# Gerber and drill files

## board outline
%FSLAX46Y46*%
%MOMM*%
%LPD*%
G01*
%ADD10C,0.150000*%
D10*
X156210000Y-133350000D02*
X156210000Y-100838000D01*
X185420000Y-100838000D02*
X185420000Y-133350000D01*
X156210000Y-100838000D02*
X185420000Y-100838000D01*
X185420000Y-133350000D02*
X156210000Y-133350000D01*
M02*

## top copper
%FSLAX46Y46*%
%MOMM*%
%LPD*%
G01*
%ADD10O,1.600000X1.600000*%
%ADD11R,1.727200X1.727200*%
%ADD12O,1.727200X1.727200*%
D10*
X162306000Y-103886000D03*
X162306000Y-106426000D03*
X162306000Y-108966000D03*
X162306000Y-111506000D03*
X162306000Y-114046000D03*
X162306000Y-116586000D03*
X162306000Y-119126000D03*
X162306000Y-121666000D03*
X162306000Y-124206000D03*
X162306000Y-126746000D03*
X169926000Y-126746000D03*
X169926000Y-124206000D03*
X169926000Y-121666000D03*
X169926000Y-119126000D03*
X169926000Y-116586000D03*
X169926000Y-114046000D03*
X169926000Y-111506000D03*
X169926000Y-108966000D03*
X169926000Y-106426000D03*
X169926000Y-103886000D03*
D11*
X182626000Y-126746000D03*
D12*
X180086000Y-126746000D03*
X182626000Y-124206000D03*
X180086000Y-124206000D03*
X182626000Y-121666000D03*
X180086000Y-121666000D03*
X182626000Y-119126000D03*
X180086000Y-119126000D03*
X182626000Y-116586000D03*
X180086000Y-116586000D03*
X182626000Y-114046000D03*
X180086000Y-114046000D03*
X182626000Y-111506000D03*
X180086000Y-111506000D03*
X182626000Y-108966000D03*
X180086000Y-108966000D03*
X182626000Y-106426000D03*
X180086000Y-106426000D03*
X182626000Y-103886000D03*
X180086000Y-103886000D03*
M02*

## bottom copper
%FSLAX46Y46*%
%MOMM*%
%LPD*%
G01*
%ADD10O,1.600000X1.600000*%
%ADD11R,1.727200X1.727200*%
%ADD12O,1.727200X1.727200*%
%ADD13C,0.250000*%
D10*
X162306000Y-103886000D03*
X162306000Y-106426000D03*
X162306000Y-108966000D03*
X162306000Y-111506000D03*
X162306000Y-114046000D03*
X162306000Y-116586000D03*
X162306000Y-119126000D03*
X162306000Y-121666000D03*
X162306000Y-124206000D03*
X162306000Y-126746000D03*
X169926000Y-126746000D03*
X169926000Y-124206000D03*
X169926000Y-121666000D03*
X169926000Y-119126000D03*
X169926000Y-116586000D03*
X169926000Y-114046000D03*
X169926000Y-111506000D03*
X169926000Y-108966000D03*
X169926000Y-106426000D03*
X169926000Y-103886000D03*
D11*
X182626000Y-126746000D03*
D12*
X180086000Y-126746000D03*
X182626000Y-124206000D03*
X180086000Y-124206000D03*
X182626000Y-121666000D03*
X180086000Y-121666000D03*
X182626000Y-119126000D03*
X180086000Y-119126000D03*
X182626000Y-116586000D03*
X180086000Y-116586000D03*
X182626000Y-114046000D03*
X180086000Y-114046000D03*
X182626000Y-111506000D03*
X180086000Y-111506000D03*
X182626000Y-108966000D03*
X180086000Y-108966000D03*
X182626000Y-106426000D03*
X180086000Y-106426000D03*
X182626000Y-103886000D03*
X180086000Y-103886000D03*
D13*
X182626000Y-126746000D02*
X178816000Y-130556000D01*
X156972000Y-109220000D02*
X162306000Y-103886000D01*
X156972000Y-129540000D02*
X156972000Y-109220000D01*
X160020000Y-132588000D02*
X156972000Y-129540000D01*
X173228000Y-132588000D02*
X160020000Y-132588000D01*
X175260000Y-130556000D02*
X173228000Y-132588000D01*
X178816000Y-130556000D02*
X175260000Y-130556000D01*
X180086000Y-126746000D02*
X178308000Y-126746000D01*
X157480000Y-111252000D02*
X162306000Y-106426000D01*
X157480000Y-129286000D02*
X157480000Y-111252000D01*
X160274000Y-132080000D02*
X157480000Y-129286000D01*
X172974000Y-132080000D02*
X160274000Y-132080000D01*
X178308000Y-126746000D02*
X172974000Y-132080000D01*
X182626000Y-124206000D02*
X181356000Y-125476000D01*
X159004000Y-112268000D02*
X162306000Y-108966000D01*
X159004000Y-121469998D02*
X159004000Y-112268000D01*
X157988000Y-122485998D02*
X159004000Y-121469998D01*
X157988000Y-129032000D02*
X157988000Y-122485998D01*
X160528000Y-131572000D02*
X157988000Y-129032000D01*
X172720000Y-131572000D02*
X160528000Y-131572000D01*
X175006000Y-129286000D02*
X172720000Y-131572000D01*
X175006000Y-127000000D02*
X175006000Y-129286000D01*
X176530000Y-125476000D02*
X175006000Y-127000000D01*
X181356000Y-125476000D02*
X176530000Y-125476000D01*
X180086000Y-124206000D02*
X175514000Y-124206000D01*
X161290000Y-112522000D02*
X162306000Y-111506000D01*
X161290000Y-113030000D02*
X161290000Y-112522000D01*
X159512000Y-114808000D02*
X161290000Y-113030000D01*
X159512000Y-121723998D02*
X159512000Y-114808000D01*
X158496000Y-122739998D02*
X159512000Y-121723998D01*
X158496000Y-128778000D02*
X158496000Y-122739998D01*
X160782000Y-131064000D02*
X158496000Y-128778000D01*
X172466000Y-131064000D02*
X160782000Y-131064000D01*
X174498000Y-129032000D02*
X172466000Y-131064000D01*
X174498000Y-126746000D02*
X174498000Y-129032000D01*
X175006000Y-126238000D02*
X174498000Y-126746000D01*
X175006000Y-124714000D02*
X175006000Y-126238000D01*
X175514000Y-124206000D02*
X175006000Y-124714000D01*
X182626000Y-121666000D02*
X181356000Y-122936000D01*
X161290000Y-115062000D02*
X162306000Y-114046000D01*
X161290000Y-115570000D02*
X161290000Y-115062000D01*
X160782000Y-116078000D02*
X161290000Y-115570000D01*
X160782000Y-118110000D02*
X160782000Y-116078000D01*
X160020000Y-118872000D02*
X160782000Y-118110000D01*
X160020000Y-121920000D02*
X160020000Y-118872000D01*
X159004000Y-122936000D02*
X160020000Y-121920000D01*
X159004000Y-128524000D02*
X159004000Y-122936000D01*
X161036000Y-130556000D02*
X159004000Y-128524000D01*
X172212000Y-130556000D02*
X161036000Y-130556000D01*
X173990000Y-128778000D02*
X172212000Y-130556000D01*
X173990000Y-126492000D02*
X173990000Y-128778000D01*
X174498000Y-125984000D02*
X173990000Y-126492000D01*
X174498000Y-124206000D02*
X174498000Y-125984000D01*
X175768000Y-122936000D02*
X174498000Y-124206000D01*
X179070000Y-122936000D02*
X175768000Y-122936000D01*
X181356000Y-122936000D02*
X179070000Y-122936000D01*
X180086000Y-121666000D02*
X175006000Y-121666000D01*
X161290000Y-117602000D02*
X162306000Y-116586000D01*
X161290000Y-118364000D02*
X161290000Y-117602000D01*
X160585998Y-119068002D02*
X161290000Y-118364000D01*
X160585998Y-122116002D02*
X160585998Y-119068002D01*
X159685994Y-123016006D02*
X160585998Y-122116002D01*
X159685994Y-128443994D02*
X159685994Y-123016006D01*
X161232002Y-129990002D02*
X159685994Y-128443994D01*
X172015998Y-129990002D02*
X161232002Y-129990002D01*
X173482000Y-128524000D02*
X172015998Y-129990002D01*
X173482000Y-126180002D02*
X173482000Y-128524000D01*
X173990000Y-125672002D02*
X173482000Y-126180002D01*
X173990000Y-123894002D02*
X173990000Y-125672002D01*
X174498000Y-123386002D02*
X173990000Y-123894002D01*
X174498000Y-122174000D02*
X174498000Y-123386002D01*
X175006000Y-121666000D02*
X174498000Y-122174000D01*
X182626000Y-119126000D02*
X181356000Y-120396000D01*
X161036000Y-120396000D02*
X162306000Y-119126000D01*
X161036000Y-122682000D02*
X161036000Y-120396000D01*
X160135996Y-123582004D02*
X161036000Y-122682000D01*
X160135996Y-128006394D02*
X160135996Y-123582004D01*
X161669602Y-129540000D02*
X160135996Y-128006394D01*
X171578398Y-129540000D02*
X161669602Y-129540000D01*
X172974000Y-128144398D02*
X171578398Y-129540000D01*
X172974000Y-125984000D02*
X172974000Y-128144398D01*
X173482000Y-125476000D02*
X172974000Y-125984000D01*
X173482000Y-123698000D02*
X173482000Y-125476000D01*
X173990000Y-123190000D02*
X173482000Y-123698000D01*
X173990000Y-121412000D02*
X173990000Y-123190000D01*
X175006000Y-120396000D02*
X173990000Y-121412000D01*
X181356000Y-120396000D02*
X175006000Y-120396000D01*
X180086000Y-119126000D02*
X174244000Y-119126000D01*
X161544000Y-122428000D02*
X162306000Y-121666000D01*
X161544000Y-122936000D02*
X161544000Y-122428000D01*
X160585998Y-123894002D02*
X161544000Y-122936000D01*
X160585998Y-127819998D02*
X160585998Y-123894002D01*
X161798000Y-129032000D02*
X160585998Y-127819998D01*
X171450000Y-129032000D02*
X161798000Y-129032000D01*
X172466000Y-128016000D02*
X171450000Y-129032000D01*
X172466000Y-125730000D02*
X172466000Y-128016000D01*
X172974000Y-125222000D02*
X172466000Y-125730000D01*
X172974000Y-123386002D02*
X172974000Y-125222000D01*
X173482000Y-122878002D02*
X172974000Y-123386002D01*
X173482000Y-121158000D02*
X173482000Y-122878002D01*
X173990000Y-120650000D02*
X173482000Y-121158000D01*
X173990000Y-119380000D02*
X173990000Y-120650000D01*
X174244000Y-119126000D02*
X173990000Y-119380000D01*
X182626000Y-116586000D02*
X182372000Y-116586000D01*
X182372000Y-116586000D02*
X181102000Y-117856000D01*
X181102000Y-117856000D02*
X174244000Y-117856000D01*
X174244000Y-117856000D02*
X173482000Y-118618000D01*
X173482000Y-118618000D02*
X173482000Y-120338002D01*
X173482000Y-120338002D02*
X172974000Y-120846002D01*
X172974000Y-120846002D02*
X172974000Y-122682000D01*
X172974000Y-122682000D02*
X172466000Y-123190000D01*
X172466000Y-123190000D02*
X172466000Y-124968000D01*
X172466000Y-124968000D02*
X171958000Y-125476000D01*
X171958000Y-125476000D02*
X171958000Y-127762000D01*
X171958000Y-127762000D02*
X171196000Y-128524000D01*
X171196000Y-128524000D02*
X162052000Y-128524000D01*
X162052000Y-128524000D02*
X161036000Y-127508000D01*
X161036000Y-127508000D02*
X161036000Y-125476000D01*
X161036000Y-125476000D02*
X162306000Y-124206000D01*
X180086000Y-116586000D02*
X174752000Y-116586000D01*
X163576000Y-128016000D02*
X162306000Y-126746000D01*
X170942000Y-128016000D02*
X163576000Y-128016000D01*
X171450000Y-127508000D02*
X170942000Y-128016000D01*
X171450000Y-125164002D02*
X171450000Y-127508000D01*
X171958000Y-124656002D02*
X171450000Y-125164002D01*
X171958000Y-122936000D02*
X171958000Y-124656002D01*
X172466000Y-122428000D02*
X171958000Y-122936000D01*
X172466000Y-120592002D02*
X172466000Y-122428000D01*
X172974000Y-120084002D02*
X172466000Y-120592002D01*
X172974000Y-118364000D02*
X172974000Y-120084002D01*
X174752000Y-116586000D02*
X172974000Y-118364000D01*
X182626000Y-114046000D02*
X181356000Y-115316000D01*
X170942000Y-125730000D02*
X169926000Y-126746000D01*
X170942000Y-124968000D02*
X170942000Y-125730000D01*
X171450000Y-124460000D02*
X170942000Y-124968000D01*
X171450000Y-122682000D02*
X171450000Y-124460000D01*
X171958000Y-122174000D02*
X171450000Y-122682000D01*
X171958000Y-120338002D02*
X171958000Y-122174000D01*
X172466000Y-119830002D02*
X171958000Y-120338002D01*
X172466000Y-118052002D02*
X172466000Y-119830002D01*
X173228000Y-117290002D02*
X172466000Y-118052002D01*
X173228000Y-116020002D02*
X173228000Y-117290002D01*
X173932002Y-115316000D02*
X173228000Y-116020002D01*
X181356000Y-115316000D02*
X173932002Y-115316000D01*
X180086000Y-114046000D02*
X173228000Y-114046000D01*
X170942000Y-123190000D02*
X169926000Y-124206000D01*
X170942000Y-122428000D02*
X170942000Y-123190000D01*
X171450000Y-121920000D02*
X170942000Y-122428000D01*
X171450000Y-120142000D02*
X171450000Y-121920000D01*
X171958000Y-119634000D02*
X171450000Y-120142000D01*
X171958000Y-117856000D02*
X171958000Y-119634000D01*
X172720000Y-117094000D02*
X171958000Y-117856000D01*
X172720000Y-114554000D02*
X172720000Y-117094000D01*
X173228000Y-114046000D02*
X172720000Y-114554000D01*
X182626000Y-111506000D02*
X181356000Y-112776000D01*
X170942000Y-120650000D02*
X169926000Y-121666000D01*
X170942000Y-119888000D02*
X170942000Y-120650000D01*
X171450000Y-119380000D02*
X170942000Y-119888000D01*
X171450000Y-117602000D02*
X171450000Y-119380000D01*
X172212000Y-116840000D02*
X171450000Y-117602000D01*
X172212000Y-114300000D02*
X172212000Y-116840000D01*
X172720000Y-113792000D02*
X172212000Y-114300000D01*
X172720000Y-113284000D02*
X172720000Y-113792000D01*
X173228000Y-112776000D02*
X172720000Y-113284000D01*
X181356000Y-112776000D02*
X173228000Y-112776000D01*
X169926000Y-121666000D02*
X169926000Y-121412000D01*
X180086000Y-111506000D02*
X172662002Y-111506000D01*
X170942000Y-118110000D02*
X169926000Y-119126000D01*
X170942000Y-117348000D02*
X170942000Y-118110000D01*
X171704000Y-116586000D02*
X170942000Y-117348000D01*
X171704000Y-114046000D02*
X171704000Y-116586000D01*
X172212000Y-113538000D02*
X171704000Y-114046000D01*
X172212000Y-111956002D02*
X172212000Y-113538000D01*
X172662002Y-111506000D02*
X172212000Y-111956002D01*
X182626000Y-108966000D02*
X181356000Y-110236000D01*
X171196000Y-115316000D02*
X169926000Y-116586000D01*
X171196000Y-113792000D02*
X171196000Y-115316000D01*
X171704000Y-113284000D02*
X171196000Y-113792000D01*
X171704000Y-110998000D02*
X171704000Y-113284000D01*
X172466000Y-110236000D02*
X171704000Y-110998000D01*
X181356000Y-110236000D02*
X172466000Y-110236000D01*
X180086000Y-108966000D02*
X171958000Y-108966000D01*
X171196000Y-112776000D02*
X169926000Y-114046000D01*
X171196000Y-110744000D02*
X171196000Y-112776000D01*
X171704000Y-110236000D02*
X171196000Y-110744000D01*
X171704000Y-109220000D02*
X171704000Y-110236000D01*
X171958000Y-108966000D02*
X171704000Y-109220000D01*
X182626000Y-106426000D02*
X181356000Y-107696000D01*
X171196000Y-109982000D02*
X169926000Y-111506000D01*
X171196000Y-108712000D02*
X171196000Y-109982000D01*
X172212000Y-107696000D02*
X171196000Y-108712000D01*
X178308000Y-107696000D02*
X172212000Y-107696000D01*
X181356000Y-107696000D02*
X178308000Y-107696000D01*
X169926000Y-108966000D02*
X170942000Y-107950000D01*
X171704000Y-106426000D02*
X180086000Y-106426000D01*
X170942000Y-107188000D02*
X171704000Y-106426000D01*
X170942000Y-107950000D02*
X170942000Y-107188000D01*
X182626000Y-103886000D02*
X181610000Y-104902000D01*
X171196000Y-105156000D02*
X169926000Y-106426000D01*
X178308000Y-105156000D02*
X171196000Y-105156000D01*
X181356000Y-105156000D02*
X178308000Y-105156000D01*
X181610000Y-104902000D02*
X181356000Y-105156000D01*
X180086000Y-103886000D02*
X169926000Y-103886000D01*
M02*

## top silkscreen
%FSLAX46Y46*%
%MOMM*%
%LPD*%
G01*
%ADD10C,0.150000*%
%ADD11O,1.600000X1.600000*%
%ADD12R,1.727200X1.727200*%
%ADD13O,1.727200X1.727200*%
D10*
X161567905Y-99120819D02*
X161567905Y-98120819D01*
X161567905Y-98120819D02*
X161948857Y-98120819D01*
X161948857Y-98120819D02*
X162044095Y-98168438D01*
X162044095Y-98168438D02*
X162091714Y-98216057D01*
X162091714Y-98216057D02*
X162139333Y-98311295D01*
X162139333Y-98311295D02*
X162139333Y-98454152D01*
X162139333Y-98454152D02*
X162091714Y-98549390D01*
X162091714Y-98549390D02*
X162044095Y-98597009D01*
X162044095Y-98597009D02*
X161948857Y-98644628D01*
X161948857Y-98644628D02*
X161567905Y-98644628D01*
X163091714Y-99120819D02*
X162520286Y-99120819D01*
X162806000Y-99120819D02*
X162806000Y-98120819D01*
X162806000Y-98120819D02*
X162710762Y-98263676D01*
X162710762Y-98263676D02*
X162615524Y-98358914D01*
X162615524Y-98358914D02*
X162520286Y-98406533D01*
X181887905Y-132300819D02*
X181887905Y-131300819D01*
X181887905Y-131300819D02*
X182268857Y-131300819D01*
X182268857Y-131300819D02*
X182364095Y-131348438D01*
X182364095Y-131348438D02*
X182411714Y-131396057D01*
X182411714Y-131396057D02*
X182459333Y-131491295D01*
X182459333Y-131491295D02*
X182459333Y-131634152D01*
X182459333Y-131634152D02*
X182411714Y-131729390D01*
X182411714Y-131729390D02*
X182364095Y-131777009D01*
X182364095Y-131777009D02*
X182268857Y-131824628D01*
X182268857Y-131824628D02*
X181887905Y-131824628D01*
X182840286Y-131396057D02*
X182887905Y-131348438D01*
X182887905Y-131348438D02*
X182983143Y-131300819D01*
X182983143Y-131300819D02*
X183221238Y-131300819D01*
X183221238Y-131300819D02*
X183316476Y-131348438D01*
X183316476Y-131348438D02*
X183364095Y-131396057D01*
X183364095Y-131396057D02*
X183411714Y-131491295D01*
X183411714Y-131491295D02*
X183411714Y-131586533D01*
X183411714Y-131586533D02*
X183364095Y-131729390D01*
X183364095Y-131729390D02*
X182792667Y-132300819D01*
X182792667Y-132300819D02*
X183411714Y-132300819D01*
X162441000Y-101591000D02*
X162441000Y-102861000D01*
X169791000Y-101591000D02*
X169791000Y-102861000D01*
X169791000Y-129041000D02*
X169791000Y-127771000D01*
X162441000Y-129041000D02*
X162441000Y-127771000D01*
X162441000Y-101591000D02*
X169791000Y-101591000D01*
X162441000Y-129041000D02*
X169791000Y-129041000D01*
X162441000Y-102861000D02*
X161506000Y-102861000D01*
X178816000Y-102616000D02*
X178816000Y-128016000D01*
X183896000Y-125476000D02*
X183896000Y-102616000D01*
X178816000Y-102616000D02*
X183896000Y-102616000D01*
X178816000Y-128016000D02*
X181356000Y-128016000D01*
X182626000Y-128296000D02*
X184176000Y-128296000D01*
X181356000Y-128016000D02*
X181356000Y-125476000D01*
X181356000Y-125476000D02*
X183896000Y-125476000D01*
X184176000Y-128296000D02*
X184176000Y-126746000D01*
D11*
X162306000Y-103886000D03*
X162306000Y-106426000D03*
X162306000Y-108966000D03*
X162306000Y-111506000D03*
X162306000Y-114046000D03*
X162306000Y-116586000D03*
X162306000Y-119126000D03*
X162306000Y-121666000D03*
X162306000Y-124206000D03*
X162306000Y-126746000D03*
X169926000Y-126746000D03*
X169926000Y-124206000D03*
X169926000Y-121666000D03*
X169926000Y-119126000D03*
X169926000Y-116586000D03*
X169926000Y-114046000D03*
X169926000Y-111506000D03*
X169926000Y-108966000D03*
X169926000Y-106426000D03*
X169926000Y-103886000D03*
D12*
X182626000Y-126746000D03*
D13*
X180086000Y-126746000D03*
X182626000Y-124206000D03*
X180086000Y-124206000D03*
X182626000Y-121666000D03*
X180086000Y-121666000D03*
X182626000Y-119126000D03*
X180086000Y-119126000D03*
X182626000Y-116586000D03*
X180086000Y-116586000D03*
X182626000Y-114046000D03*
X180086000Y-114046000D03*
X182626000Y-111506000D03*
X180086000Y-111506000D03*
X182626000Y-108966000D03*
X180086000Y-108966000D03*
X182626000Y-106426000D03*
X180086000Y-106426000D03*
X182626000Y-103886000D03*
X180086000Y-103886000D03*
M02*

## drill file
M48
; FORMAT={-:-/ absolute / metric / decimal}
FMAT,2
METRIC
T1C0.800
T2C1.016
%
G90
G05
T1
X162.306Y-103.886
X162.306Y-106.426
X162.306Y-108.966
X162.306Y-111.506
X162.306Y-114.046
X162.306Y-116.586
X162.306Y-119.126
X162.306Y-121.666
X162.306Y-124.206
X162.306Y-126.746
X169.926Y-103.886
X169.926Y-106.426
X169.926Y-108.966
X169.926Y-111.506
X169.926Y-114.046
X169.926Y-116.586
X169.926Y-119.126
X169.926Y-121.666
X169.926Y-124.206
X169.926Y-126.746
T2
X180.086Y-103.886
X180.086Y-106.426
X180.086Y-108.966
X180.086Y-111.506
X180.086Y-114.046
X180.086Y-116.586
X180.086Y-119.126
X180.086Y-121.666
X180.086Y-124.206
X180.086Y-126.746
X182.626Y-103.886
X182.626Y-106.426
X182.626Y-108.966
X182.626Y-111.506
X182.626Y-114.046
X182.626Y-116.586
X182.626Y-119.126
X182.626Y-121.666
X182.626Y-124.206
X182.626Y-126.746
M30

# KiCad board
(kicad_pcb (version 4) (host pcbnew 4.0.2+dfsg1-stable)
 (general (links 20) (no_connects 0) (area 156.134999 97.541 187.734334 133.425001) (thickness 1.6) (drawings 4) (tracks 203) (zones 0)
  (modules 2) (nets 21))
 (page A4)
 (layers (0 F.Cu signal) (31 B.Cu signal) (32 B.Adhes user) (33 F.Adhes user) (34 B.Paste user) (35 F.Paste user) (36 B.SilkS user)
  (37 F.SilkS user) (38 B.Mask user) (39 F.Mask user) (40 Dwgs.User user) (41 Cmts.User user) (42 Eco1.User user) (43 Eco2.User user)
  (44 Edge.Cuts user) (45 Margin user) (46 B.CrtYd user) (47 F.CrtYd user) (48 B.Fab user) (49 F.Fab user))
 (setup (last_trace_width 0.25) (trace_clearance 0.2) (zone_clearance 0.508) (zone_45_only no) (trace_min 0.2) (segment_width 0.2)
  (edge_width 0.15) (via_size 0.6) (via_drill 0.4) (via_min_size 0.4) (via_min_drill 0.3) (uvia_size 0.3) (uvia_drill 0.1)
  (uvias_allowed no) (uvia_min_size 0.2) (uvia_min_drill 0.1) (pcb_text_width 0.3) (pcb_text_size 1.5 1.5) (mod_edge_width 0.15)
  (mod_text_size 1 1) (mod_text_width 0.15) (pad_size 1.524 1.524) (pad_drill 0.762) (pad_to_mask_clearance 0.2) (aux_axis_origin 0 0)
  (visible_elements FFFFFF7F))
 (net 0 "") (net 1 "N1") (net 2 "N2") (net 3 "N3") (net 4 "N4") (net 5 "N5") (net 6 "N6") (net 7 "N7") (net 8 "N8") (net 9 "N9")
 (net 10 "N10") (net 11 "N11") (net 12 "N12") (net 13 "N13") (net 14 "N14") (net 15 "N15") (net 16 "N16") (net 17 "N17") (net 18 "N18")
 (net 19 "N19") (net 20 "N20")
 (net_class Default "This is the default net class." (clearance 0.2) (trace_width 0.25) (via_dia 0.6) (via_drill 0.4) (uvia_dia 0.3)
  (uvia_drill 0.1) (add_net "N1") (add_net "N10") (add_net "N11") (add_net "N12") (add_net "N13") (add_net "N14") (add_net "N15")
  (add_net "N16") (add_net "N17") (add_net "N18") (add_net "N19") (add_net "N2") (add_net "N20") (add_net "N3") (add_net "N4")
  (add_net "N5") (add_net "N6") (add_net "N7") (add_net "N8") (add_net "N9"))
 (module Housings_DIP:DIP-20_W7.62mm (layer F.Cu) (at 162.306 103.886)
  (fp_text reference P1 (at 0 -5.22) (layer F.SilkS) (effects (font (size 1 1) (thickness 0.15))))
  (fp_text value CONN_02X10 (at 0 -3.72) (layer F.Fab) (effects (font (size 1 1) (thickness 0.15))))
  (fp_line (start 0.135 -2.295) (end 0.135 -1.025) (layer F.SilkS) (width 0.15))
  (fp_line (start 7.485 -2.295) (end 7.485 -1.025) (layer F.SilkS) (width 0.15))
  (fp_line (start 7.485 25.155) (end 7.485 23.885) (layer F.SilkS) (width 0.15))
  (fp_line (start 0.135 25.155) (end 0.135 23.885) (layer F.SilkS) (width 0.15))
  (fp_line (start 0.135 -2.295) (end 7.485 -2.295) (layer F.SilkS) (width 0.15))
  (fp_line (start 0.135 25.155) (end 7.485 25.155) (layer F.SilkS) (width 0.15))
  (fp_line (start 0.135 -1.025) (end -0.8 -1.025) (layer F.SilkS) (width 0.15))
  (pad 1 thru_hole oval (at 0 0) (size 1.6 1.6) (drill 0.8) (layers *.Cu *.Mask F.SilkS) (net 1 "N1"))
  (pad 2 thru_hole oval (at 0 2.54) (size 1.6 1.6) (drill 0.8) (layers *.Cu *.Mask F.SilkS) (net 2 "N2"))
  (pad 3 thru_hole oval (at 0 5.08) (size 1.6 1.6) (drill 0.8) (layers *.Cu *.Mask F.SilkS) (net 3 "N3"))
  (pad 4 thru_hole oval (at 0 7.62) (size 1.6 1.6) (drill 0.8) (layers *.Cu *.Mask F.SilkS) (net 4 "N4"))
  (pad 5 thru_hole oval (at 0 10.16) (size 1.6 1.6) (drill 0.8) (layers *.Cu *.Mask F.SilkS) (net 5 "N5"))
  (pad 6 thru_hole oval (at 0 12.7) (size 1.6 1.6) (drill 0.8) (layers *.Cu *.Mask F.SilkS) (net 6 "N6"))
  (pad 7 thru_hole oval (at 0 15.24) (size 1.6 1.6) (drill 0.8) (layers *.Cu *.Mask F.SilkS) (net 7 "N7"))
  (pad 8 thru_hole oval (at 0 17.78) (size 1.6 1.6) (drill 0.8) (layers *.Cu *.Mask F.SilkS) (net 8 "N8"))
  (pad 9 thru_hole oval (at 0 20.32) (size 1.6 1.6) (drill 0.8) (layers *.Cu *.Mask F.SilkS) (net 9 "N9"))
  (pad 10 thru_hole oval (at 0 22.86) (size 1.6 1.6) (drill 0.8) (layers *.Cu *.Mask F.SilkS) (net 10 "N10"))
  (pad 11 thru_hole oval (at 7.62 22.86) (size 1.6 1.6) (drill 0.8) (layers *.Cu *.Mask F.SilkS) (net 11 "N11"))
  (pad 12 thru_hole oval (at 7.62 20.32) (size 1.6 1.6) (drill 0.8) (layers *.Cu *.Mask F.SilkS) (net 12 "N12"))
  (pad 13 thru_hole oval (at 7.62 17.78) (size 1.6 1.6) (drill 0.8) (layers *.Cu *.Mask F.SilkS) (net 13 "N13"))
  (pad 14 thru_hole oval (at 7.62 15.24) (size 1.6 1.6) (drill 0.8) (layers *.Cu *.Mask F.SilkS) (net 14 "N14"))
  (pad 15 thru_hole oval (at 7.62 12.7) (size 1.6 1.6) (drill 0.8) (layers *.Cu *.Mask F.SilkS) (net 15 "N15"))
  (pad 16 thru_hole oval (at 7.62 10.16) (size 1.6 1.6) (drill 0.8) (layers *.Cu *.Mask F.SilkS) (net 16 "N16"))
  (pad 17 thru_hole oval (at 7.62 7.62) (size 1.6 1.6) (drill 0.8) (layers *.Cu *.Mask F.SilkS) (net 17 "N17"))
  (pad 18 thru_hole oval (at 7.62 5.08) (size 1.6 1.6) (drill 0.8) (layers *.Cu *.Mask F.SilkS) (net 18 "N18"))
  (pad 19 thru_hole oval (at 7.62 2.54) (size 1.6 1.6) (drill 0.8) (layers *.Cu *.Mask F.SilkS) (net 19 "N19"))
  (pad 20 thru_hole oval (at 7.62 0) (size 1.6 1.6) (drill 0.8) (layers *.Cu *.Mask F.SilkS) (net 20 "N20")))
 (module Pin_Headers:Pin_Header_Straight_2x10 (layer F.Cu) (at 182.626 126.746 180)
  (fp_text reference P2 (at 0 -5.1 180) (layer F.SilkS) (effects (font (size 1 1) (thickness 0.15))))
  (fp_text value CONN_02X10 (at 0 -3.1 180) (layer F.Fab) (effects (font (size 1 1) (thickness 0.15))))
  (fp_line (start 3.81 24.13) (end 3.81 -1.27) (layer F.SilkS) (width 0.15))
  (fp_line (start -1.27 1.27) (end -1.27 24.13) (layer F.SilkS) (width 0.15))
  (fp_line (start 3.81 24.13) (end -1.27 24.13) (layer F.SilkS) (width 0.15))
  (fp_line (start 3.81 -1.27) (end 1.27 -1.27) (layer F.SilkS) (width 0.15))
  (fp_line (start 0 -1.55) (end -1.55 -1.55) (layer F.SilkS) (width 0.15))
  (fp_line (start 1.27 -1.27) (end 1.27 1.27) (layer F.SilkS) (width 0.15))
  (fp_line (start 1.27 1.27) (end -1.27 1.27) (layer F.SilkS) (width 0.15))
  (fp_line (start -1.55 -1.55) (end -1.55 0) (layer F.SilkS) (width 0.15))
  (pad 1 thru_hole rect (at 0 0 180) (size 1.7272 1.7272) (drill 1.016) (layers *.Cu *.Mask F.SilkS) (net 1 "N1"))
  (pad 2 thru_hole oval (at 2.54 0 180) (size 1.7272 1.7272) (drill 1.016) (layers *.Cu *.Mask F.SilkS) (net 2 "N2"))
  (pad 3 thru_hole oval (at 0 2.54 180) (size 1.7272 1.7272) (drill 1.016) (layers *.Cu *.Mask F.SilkS) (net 3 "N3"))
  (pad 4 thru_hole oval (at 2.54 2.54 180) (size 1.7272 1.7272) (drill 1.016) (layers *.Cu *.Mask F.SilkS) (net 4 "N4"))
  (pad 5 thru_hole oval (at 0 5.08 180) (size 1.7272 1.7272) (drill 1.016) (layers *.Cu *.Mask F.SilkS) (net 5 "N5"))
  (pad 6 thru_hole oval (at 2.54 5.08 180) (size 1.7272 1.7272) (drill 1.016) (layers *.Cu *.Mask F.SilkS) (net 6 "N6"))
  (pad 7 thru_hole oval (at 0 7.62 180) (size 1.7272 1.7272) (drill 1.016) (layers *.Cu *.Mask F.SilkS) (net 7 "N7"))
  (pad 8 thru_hole oval (at 2.54 7.62 180) (size 1.7272 1.7272) (drill 1.016) (layers *.Cu *.Mask F.SilkS) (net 8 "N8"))
  (pad 9 thru_hole oval (at 0 10.16 180) (size 1.7272 1.7272) (drill 1.016) (layers *.Cu *.Mask F.SilkS) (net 9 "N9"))
  (pad 10 thru_hole oval (at 2.54 10.16 180) (size 1.7272 1.7272) (drill 1.016) (layers *.Cu *.Mask F.SilkS) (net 10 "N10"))
  (pad 11 thru_hole oval (at 0 12.7 180) (size 1.7272 1.7272) (drill 1.016) (layers *.Cu *.Mask F.SilkS) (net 11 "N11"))
  (pad 12 thru_hole oval (at 2.54 12.7 180) (size 1.7272 1.7272) (drill 1.016) (layers *.Cu *.Mask F.SilkS) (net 12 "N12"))
  (pad 13 thru_hole oval (at 0 15.24 180) (size 1.7272 1.7272) (drill 1.016) (layers *.Cu *.Mask F.SilkS) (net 13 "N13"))
  (pad 14 thru_hole oval (at 2.54 15.24 180) (size 1.7272 1.7272) (drill 1.016) (layers *.Cu *.Mask F.SilkS) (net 14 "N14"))
  (pad 15 thru_hole oval (at 0 17.78 180) (size 1.7272 1.7272) (drill 1.016) (layers *.Cu *.Mask F.SilkS) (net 15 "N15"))
  (pad 16 thru_hole oval (at 2.54 17.78 180) (size 1.7272 1.7272) (drill 1.016) (layers *.Cu *.Mask F.SilkS) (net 16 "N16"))
  (pad 17 thru_hole oval (at 0 20.32 180) (size 1.7272 1.7272) (drill 1.016) (layers *.Cu *.Mask F.SilkS) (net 17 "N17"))
  (pad 18 thru_hole oval (at 2.54 20.32 180) (size 1.7272 1.7272) (drill 1.016) (layers *.Cu *.Mask F.SilkS) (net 18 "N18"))
  (pad 19 thru_hole oval (at 0 22.86 180) (size 1.7272 1.7272) (drill 1.016) (layers *.Cu *.Mask F.SilkS) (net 19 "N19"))
  (pad 20 thru_hole oval (at 2.54 22.86 180) (size 1.7272 1.7272) (drill 1.016) (layers *.Cu *.Mask F.SilkS) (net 20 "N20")))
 (gr_line (start 156.21 133.35) (end 156.21 100.838) (angle 90) (layer Edge.Cuts) (width 0.15))
 (gr_line (start 185.42 100.838) (end 185.42 133.35) (angle 90) (layer Edge.Cuts) (width 0.15))
 (gr_line (start 156.21 100.838) (end 185.42 100.838) (angle 90) (layer Edge.Cuts) (width 0.15))
 (gr_line (start 185.42 133.35) (end 156.21 133.35) (angle 90) (layer Edge.Cuts) (width 0.15))
 (segment (start 182.626 126.746) (end 178.816 130.556) (width 0.25) (layer B.Cu) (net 1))
 (segment (start 156.972 109.22) (end 162.306 103.886) (width 0.25) (layer B.Cu) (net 1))
 (segment (start 156.972 129.54) (end 156.972 109.22) (width 0.25) (layer B.Cu) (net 1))
 (segment (start 160.02 132.588) (end 156.972 129.54) (width 0.25) (layer B.Cu) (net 1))
 (segment (start 173.228 132.588) (end 160.02 132.588) (width 0.25) (layer B.Cu) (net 1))
 (segment (start 175.26 130.556) (end 173.228 132.588) (width 0.25) (layer B.Cu) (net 1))
 (segment (start 178.816 130.556) (end 175.26 130.556) (width 0.25) (layer B.Cu) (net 1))
 (segment (start 180.086 126.746) (end 178.308 126.746) (width 0.25) (layer B.Cu) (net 2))
 (segment (start 157.48 111.252) (end 162.306 106.426) (width 0.25) (layer B.Cu) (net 2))
 (segment (start 157.48 129.286) (end 157.48 111.252) (width 0.25) (layer B.Cu) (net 2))
 (segment (start 160.274 132.08) (end 157.48 129.286) (width 0.25) (layer B.Cu) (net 2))
 (segment (start 172.974 132.08) (end 160.274 132.08) (width 0.25) (layer B.Cu) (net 2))
 (segment (start 178.308 126.746) (end 172.974 132.08) (width 0.25) (layer B.Cu) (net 2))
 (segment (start 182.626 124.206) (end 181.356 125.476) (width 0.25) (layer B.Cu) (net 3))
 (segment (start 159.004 112.268) (end 162.306 108.966) (width 0.25) (layer B.Cu) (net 3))
 (segment (start 159.004 121.469998) (end 159.004 112.268) (width 0.25) (layer B.Cu) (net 3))
 (segment (start 157.988 122.485998) (end 159.004 121.469998) (width 0.25) (layer B.Cu) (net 3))
 (segment (start 157.988 129.032) (end 157.988 122.485998) (width 0.25) (layer B.Cu) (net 3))
 (segment (start 160.528 131.572) (end 157.988 129.032) (width 0.25) (layer B.Cu) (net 3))
 (segment (start 172.72 131.572) (end 160.528 131.572) (width 0.25) (layer B.Cu) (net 3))
 (segment (start 175.006 129.286) (end 172.72 131.572) (width 0.25) (layer B.Cu) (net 3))
 (segment (start 175.006 127) (end 175.006 129.286) (width 0.25) (layer B.Cu) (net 3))
 (segment (start 176.53 125.476) (end 175.006 127) (width 0.25) (layer B.Cu) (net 3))
 (segment (start 181.356 125.476) (end 176.53 125.476) (width 0.25) (layer B.Cu) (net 3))
 (segment (start 180.086 124.206) (end 175.514 124.206) (width 0.25) (layer B.Cu) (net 4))
 (segment (start 161.29 112.522) (end 162.306 111.506) (width 0.25) (layer B.Cu) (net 4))
 (segment (start 161.29 113.03) (end 161.29 112.522) (width 0.25) (layer B.Cu) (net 4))
 (segment (start 159.512 114.808) (end 161.29 113.03) (width 0.25) (layer B.Cu) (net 4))
 (segment (start 159.512 121.723998) (end 159.512 114.808) (width 0.25) (layer B.Cu) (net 4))
 (segment (start 158.496 122.739998) (end 159.512 121.723998) (width 0.25) (layer B.Cu) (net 4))
 (segment (start 158.496 128.778) (end 158.496 122.739998) (width 0.25) (layer B.Cu) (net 4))
 (segment (start 160.782 131.064) (end 158.496 128.778) (width 0.25) (layer B.Cu) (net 4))
 (segment (start 172.466 131.064) (end 160.782 131.064) (width 0.25) (layer B.Cu) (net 4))
 (segment (start 174.498 129.032) (end 172.466 131.064) (width 0.25) (layer B.Cu) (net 4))
 (segment (start 174.498 126.746) (end 174.498 129.032) (width 0.25) (layer B.Cu) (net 4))
 (segment (start 175.006 126.238) (end 174.498 126.746) (width 0.25) (layer B.Cu) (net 4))
 (segment (start 175.006 124.714) (end 175.006 126.238) (width 0.25) (layer B.Cu) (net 4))
 (segment (start 175.514 124.206) (end 175.006 124.714) (width 0.25) (layer B.Cu) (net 4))
 (segment (start 182.626 121.666) (end 181.356 122.936) (width 0.25) (layer B.Cu) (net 5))
 (segment (start 161.29 115.062) (end 162.306 114.046) (width 0.25) (layer B.Cu) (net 5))
 (segment (start 161.29 115.57) (end 161.29 115.062) (width 0.25) (layer B.Cu) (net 5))
 (segment (start 160.782 116.078) (end 161.29 115.57) (width 0.25) (layer B.Cu) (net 5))
 (segment (start 160.782 118.11) (end 160.782 116.078) (width 0.25) (layer B.Cu) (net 5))
 (segment (start 160.02 118.872) (end 160.782 118.11) (width 0.25) (layer B.Cu) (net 5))
 (segment (start 160.02 121.92) (end 160.02 118.872) (width 0.25) (layer B.Cu) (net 5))
 (segment (start 159.004 122.936) (end 160.02 121.92) (width 0.25) (layer B.Cu) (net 5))
 (segment (start 159.004 128.524) (end 159.004 122.936) (width 0.25) (layer B.Cu) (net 5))
 (segment (start 161.036 130.556) (end 159.004 128.524) (width 0.25) (layer B.Cu) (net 5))
 (segment (start 172.212 130.556) (end 161.036 130.556) (width 0.25) (layer B.Cu) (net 5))
 (segment (start 173.99 128.778) (end 172.212 130.556) (width 0.25) (layer B.Cu) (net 5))
 (segment (start 173.99 126.492) (end 173.99 128.778) (width 0.25) (layer B.Cu) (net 5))
 (segment (start 174.498 125.984) (end 173.99 126.492) (width 0.25) (layer B.Cu) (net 5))
 (segment (start 174.498 124.206) (end 174.498 125.984) (width 0.25) (layer B.Cu) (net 5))
 (segment (start 175.768 122.936) (end 174.498 124.206) (width 0.25) (layer B.Cu) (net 5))
 (segment (start 179.07 122.936) (end 175.768 122.936) (width 0.25) (layer B.Cu) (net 5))
 (segment (start 181.356 122.936) (end 179.07 122.936) (width 0.25) (layer B.Cu) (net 5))
 (segment (start 180.086 121.666) (end 175.006 121.666) (width 0.25) (layer B.Cu) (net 6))
 (segment (start 161.29 117.602) (end 162.306 116.586) (width 0.25) (layer B.Cu) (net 6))
 (segment (start 161.29 118.364) (end 161.29 117.602) (width 0.25) (layer B.Cu) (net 6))
 (segment (start 160.585998 119.068002) (end 161.29 118.364) (width 0.25) (layer B.Cu) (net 6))
 (segment (start 160.585998 122.116002) (end 160.585998 119.068002) (width 0.25) (layer B.Cu) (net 6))
 (segment (start 159.685994 123.016006) (end 160.585998 122.116002) (width 0.25) (layer B.Cu) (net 6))
 (segment (start 159.685994 128.443994) (end 159.685994 123.016006) (width 0.25) (layer B.Cu) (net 6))
 (segment (start 161.232002 129.990002) (end 159.685994 128.443994) (width 0.25) (layer B.Cu) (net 6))
 (segment (start 172.015998 129.990002) (end 161.232002 129.990002) (width 0.25) (layer B.Cu) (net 6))
 (segment (start 173.482 128.524) (end 172.015998 129.990002) (width 0.25) (layer B.Cu) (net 6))
 (segment (start 173.482 126.180002) (end 173.482 128.524) (width 0.25) (layer B.Cu) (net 6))
 (segment (start 173.99 125.672002) (end 173.482 126.180002) (width 0.25) (layer B.Cu) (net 6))
 (segment (start 173.99 123.894002) (end 173.99 125.672002) (width 0.25) (layer B.Cu) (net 6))
 (segment (start 174.498 123.386002) (end 173.99 123.894002) (width 0.25) (layer B.Cu) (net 6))
 (segment (start 174.498 122.174) (end 174.498 123.386002) (width 0.25) (layer B.Cu) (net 6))
 (segment (start 175.006 121.666) (end 174.498 122.174) (width 0.25) (layer B.Cu) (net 6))
 (segment (start 182.626 119.126) (end 181.356 120.396) (width 0.25) (layer B.Cu) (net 7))
 (segment (start 161.036 120.396) (end 162.306 119.126) (width 0.25) (layer B.Cu) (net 7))
 (segment (start 161.036 122.682) (end 161.036 120.396) (width 0.25) (layer B.Cu) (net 7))
 (segment (start 160.135996 123.582004) (end 161.036 122.682) (width 0.25) (layer B.Cu) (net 7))
 (segment (start 160.135996 128.006394) (end 160.135996 123.582004) (width 0.25) (layer B.Cu) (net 7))
 (segment (start 161.669602 129.54) (end 160.135996 128.006394) (width 0.25) (layer B.Cu) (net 7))
 (segment (start 171.578398 129.54) (end 161.669602 129.54) (width 0.25) (layer B.Cu) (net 7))
 (segment (start 172.974 128.144398) (end 171.578398 129.54) (width 0.25) (layer B.Cu) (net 7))
 (segment (start 172.974 125.984) (end 172.974 128.144398) (width 0.25) (layer B.Cu) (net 7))
 (segment (start 173.482 125.476) (end 172.974 125.984) (width 0.25) (layer B.Cu) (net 7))
 (segment (start 173.482 123.698) (end 173.482 125.476) (width 0.25) (layer B.Cu) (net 7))
 (segment (start 173.99 123.19) (end 173.482 123.698) (width 0.25) (layer B.Cu) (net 7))
 (segment (start 173.99 121.412) (end 173.99 123.19) (width 0.25) (layer B.Cu) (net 7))
 (segment (start 175.006 120.396) (end 173.99 121.412) (width 0.25) (layer B.Cu) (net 7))
 (segment (start 181.356 120.396) (end 175.006 120.396) (width 0.25) (layer B.Cu) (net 7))
 (segment (start 180.086 119.126) (end 174.244 119.126) (width 0.25) (layer B.Cu) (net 8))
 (segment (start 161.544 122.428) (end 162.306 121.666) (width 0.25) (layer B.Cu) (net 8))
 (segment (start 161.544 122.936) (end 161.544 122.428) (width 0.25) (layer B.Cu) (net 8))
 (segment (start 160.585998 123.894002) (end 161.544 122.936) (width 0.25) (layer B.Cu) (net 8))
 (segment (start 160.585998 127.819998) (end 160.585998 123.894002) (width 0.25) (layer B.Cu) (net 8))
 (segment (start 161.798 129.032) (end 160.585998 127.819998) (width 0.25) (layer B.Cu) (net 8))
 (segment (start 171.45 129.032) (end 161.798 129.032) (width 0.25) (layer B.Cu) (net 8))
 (segment (start 172.466 128.016) (end 171.45 129.032) (width 0.25) (layer B.Cu) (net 8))
 (segment (start 172.466 125.73) (end 172.466 128.016) (width 0.25) (layer B.Cu) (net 8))
 (segment (start 172.974 125.222) (end 172.466 125.73) (width 0.25) (layer B.Cu) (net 8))
 (segment (start 172.974 123.386002) (end 172.974 125.222) (width 0.25) (layer B.Cu) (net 8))
 (segment (start 173.482 122.878002) (end 172.974 123.386002) (width 0.25) (layer B.Cu) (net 8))
 (segment (start 173.482 121.158) (end 173.482 122.878002) (width 0.25) (layer B.Cu) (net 8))
 (segment (start 173.99 120.65) (end 173.482 121.158) (width 0.25) (layer B.Cu) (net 8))
 (segment (start 173.99 119.38) (end 173.99 120.65) (width 0.25) (layer B.Cu) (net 8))
 (segment (start 174.244 119.126) (end 173.99 119.38) (width 0.25) (layer B.Cu) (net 8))
 (segment (start 182.626 116.586) (end 182.372 116.586) (width 0.25) (layer B.Cu) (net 9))
 (segment (start 182.372 116.586) (end 181.102 117.856) (width 0.25) (layer B.Cu) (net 9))
 (segment (start 181.102 117.856) (end 174.244 117.856) (width 0.25) (layer B.Cu) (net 9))
 (segment (start 174.244 117.856) (end 173.482 118.618) (width 0.25) (layer B.Cu) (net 9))
 (segment (start 173.482 118.618) (end 173.482 120.338002) (width 0.25) (layer B.Cu) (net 9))
 (segment (start 173.482 120.338002) (end 172.974 120.846002) (width 0.25) (layer B.Cu) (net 9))
 (segment (start 172.974 120.846002) (end 172.974 122.682) (width 0.25) (layer B.Cu) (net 9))
 (segment (start 172.974 122.682) (end 172.466 123.19) (width 0.25) (layer B.Cu) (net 9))
 (segment (start 172.466 123.19) (end 172.466 124.968) (width 0.25) (layer B.Cu) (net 9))
 (segment (start 172.466 124.968) (end 171.958 125.476) (width 0.25) (layer B.Cu) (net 9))
 (segment (start 171.958 125.476) (end 171.958 127.762) (width 0.25) (layer B.Cu) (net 9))
 (segment (start 171.958 127.762) (end 171.196 128.524) (width 0.25) (layer B.Cu) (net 9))
 (segment (start 171.196 128.524) (end 162.052 128.524) (width 0.25) (layer B.Cu) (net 9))
 (segment (start 162.052 128.524) (end 161.036 127.508) (width 0.25) (layer B.Cu) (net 9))
 (segment (start 161.036 127.508) (end 161.036 125.476) (width 0.25) (layer B.Cu) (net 9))
 (segment (start 161.036 125.476) (end 162.306 124.206) (width 0.25) (layer B.Cu) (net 9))
 (segment (start 180.086 116.586) (end 174.752 116.586) (width 0.25) (layer B.Cu) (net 10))
 (segment (start 163.576 128.016) (end 162.306 126.746) (width 0.25) (layer B.Cu) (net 10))
 (segment (start 170.942 128.016) (end 163.576 128.016) (width 0.25) (layer B.Cu) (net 10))
 (segment (start 171.45 127.508) (end 170.942 128.016) (width 0.25) (layer B.Cu) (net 10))
 (segment (start 171.45 125.164002) (end 171.45 127.508) (width 0.25) (layer B.Cu) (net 10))
 (segment (start 171.958 124.656002) (end 171.45 125.164002) (width 0.25) (layer B.Cu) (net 10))
 (segment (start 171.958 122.936) (end 171.958 124.656002) (width 0.25) (layer B.Cu) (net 10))
 (segment (start 172.466 122.428) (end 171.958 122.936) (width 0.25) (layer B.Cu) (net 10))
 (segment (start 172.466 120.592002) (end 172.466 122.428) (width 0.25) (layer B.Cu) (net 10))
 (segment (start 172.974 120.084002) (end 172.466 120.592002) (width 0.25) (layer B.Cu) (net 10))
 (segment (start 172.974 118.364) (end 172.974 120.084002) (width 0.25) (layer B.Cu) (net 10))
 (segment (start 174.752 116.586) (end 172.974 118.364) (width 0.25) (layer B.Cu) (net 10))
 (segment (start 182.626 114.046) (end 181.356 115.316) (width 0.25) (layer B.Cu) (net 11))
 (segment (start 170.942 125.73) (end 169.926 126.746) (width 0.25) (layer B.Cu) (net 11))
 (segment (start 170.942 124.968) (end 170.942 125.73) (width 0.25) (layer B.Cu) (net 11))
 (segment (start 171.45 124.46) (end 170.942 124.968) (width 0.25) (layer B.Cu) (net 11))
 (segment (start 171.45 122.682) (end 171.45 124.46) (width 0.25) (layer B.Cu) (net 11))
 (segment (start 171.958 122.174) (end 171.45 122.682) (width 0.25) (layer B.Cu) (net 11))
 (segment (start 171.958 120.338002) (end 171.958 122.174) (width 0.25) (layer B.Cu) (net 11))
 (segment (start 172.466 119.830002) (end 171.958 120.338002) (width 0.25) (layer B.Cu) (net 11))
 (segment (start 172.466 118.052002) (end 172.466 119.830002) (width 0.25) (layer B.Cu) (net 11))
 (segment (start 173.228 117.290002) (end 172.466 118.052002) (width 0.25) (layer B.Cu) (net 11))
 (segment (start 173.228 116.020002) (end 173.228 117.290002) (width 0.25) (layer B.Cu) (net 11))
 (segment (start 173.932002 115.316) (end 173.228 116.020002) (width 0.25) (layer B.Cu) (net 11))
 (segment (start 181.356 115.316) (end 173.932002 115.316) (width 0.25) (layer B.Cu) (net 11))
 (segment (start 180.086 114.046) (end 173.228 114.046) (width 0.25) (layer B.Cu) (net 12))
 (segment (start 170.942 123.19) (end 169.926 124.206) (width 0.25) (layer B.Cu) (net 12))
 (segment (start 170.942 122.428) (end 170.942 123.19) (width 0.25) (layer B.Cu) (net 12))
 (segment (start 171.45 121.92) (end 170.942 122.428) (width 0.25) (layer B.Cu) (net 12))
 (segment (start 171.45 120.142) (end 171.45 121.92) (width 0.25) (layer B.Cu) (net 12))
 (segment (start 171.958 119.634) (end 171.45 120.142) (width 0.25) (layer B.Cu) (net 12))
 (segment (start 171.958 117.856) (end 171.958 119.634) (width 0.25) (layer B.Cu) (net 12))
 (segment (start 172.72 117.094) (end 171.958 117.856) (width 0.25) (layer B.Cu) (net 12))
 (segment (start 172.72 114.554) (end 172.72 117.094) (width 0.25) (layer B.Cu) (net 12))
 (segment (start 173.228 114.046) (end 172.72 114.554) (width 0.25) (layer B.Cu) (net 12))
 (segment (start 182.626 111.506) (end 181.356 112.776) (width 0.25) (layer B.Cu) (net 13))
 (segment (start 170.942 120.65) (end 169.926 121.666) (width 0.25) (layer B.Cu) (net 13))
 (segment (start 170.942 119.888) (end 170.942 120.65) (width 0.25) (layer B.Cu) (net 13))
 (segment (start 171.45 119.38) (end 170.942 119.888) (width 0.25) (layer B.Cu) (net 13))
 (segment (start 171.45 117.602) (end 171.45 119.38) (width 0.25) (layer B.Cu) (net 13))
 (segment (start 172.212 116.84) (end 171.45 117.602) (width 0.25) (layer B.Cu) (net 13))
 (segment (start 172.212 114.3) (end 172.212 116.84) (width 0.25) (layer B.Cu) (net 13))
 (segment (start 172.72 113.792) (end 172.212 114.3) (width 0.25) (layer B.Cu) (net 13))
 (segment (start 172.72 113.284) (end 172.72 113.792) (width 0.25) (layer B.Cu) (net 13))
 (segment (start 173.228 112.776) (end 172.72 113.284) (width 0.25) (layer B.Cu) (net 13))
 (segment (start 181.356 112.776) (end 173.228 112.776) (width 0.25) (layer B.Cu) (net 13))
 (segment (start 169.926 121.666) (end 169.926 121.412) (width 0.25) (layer B.Cu) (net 13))
 (segment (start 180.086 111.506) (end 172.662002 111.506) (width 0.25) (layer B.Cu) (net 14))
 (segment (start 170.942 118.11) (end 169.926 119.126) (width 0.25) (layer B.Cu) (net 14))
 (segment (start 170.942 117.348) (end 170.942 118.11) (width 0.25) (layer B.Cu) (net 14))
 (segment (start 171.704 116.586) (end 170.942 117.348) (width 0.25) (layer B.Cu) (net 14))
 (segment (start 171.704 114.046) (end 171.704 116.586) (width 0.25) (layer B.Cu) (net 14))
 (segment (start 172.212 113.538) (end 171.704 114.046) (width 0.25) (layer B.Cu) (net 14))
 (segment (start 172.212 111.956002) (end 172.212 113.538) (width 0.25) (layer B.Cu) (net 14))
 (segment (start 172.662002 111.506) (end 172.212 111.956002) (width 0.25) (layer B.Cu) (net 14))
 (segment (start 182.626 108.966) (end 181.356 110.236) (width 0.25) (layer B.Cu) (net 15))
 (segment (start 171.196 115.316) (end 169.926 116.586) (width 0.25) (layer B.Cu) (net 15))
 (segment (start 171.196 113.792) (end 171.196 115.316) (width 0.25) (layer B.Cu) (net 15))
 (segment (start 171.704 113.284) (end 171.196 113.792) (width 0.25) (layer B.Cu) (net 15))
 (segment (start 171.704 110.998) (end 171.704 113.284) (width 0.25) (layer B.Cu) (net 15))
 (segment (start 172.466 110.236) (end 171.704 110.998) (width 0.25) (layer B.Cu) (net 15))
 (segment (start 181.356 110.236) (end 172.466 110.236) (width 0.25) (layer B.Cu) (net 15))
 (segment (start 180.086 108.966) (end 171.958 108.966) (width 0.25) (layer B.Cu) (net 16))
 (segment (start 171.196 112.776) (end 169.926 114.046) (width 0.25) (layer B.Cu) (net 16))
 (segment (start 171.196 110.744) (end 171.196 112.776) (width 0.25) (layer B.Cu) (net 16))
 (segment (start 171.704 110.236) (end 171.196 110.744) (width 0.25) (layer B.Cu) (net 16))
 (segment (start 171.704 109.22) (end 171.704 110.236) (width 0.25) (layer B.Cu) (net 16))
 (segment (start 171.958 108.966) (end 171.704 109.22) (width 0.25) (layer B.Cu) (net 16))
 (segment (start 182.626 106.426) (end 181.356 107.696) (width 0.25) (layer B.Cu) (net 17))
 (segment (start 171.196 109.982) (end 169.926 111.506) (width 0.25) (layer B.Cu) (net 17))
 (segment (start 171.196 108.712) (end 171.196 109.982) (width 0.25) (layer B.Cu) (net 17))
 (segment (start 172.212 107.696) (end 171.196 108.712) (width 0.25) (layer B.Cu) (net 17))
 (segment (start 178.308 107.696) (end 172.212 107.696) (width 0.25) (layer B.Cu) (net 17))
 (segment (start 181.356 107.696) (end 178.308 107.696) (width 0.25) (layer B.Cu) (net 17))
 (segment (start 169.926 108.966) (end 170.942 107.95) (width 0.25) (layer B.Cu) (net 18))
 (segment (start 171.704 106.426) (end 180.086 106.426) (width 0.25) (layer B.Cu) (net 18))
 (segment (start 170.942 107.188) (end 171.704 106.426) (width 0.25) (layer B.Cu) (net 18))
 (segment (start 170.942 107.95) (end 170.942 107.188) (width 0.25) (layer B.Cu) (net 18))
 (segment (start 182.626 103.886) (end 181.61 104.902) (width 0.25) (layer B.Cu) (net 19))
 (segment (start 171.196 105.156) (end 169.926 106.426) (width 0.25) (layer B.Cu) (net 19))
 (segment (start 178.308 105.156) (end 171.196 105.156) (width 0.25) (layer B.Cu) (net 19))
 (segment (start 181.356 105.156) (end 178.308 105.156) (width 0.25) (layer B.Cu) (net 19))
 (segment (start 181.61 104.902) (end 181.356 105.156) (width 0.25) (layer B.Cu) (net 19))
 (segment (start 180.086 103.886) (end 169.926 103.886) (width 0.25) (layer B.Cu) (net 20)))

